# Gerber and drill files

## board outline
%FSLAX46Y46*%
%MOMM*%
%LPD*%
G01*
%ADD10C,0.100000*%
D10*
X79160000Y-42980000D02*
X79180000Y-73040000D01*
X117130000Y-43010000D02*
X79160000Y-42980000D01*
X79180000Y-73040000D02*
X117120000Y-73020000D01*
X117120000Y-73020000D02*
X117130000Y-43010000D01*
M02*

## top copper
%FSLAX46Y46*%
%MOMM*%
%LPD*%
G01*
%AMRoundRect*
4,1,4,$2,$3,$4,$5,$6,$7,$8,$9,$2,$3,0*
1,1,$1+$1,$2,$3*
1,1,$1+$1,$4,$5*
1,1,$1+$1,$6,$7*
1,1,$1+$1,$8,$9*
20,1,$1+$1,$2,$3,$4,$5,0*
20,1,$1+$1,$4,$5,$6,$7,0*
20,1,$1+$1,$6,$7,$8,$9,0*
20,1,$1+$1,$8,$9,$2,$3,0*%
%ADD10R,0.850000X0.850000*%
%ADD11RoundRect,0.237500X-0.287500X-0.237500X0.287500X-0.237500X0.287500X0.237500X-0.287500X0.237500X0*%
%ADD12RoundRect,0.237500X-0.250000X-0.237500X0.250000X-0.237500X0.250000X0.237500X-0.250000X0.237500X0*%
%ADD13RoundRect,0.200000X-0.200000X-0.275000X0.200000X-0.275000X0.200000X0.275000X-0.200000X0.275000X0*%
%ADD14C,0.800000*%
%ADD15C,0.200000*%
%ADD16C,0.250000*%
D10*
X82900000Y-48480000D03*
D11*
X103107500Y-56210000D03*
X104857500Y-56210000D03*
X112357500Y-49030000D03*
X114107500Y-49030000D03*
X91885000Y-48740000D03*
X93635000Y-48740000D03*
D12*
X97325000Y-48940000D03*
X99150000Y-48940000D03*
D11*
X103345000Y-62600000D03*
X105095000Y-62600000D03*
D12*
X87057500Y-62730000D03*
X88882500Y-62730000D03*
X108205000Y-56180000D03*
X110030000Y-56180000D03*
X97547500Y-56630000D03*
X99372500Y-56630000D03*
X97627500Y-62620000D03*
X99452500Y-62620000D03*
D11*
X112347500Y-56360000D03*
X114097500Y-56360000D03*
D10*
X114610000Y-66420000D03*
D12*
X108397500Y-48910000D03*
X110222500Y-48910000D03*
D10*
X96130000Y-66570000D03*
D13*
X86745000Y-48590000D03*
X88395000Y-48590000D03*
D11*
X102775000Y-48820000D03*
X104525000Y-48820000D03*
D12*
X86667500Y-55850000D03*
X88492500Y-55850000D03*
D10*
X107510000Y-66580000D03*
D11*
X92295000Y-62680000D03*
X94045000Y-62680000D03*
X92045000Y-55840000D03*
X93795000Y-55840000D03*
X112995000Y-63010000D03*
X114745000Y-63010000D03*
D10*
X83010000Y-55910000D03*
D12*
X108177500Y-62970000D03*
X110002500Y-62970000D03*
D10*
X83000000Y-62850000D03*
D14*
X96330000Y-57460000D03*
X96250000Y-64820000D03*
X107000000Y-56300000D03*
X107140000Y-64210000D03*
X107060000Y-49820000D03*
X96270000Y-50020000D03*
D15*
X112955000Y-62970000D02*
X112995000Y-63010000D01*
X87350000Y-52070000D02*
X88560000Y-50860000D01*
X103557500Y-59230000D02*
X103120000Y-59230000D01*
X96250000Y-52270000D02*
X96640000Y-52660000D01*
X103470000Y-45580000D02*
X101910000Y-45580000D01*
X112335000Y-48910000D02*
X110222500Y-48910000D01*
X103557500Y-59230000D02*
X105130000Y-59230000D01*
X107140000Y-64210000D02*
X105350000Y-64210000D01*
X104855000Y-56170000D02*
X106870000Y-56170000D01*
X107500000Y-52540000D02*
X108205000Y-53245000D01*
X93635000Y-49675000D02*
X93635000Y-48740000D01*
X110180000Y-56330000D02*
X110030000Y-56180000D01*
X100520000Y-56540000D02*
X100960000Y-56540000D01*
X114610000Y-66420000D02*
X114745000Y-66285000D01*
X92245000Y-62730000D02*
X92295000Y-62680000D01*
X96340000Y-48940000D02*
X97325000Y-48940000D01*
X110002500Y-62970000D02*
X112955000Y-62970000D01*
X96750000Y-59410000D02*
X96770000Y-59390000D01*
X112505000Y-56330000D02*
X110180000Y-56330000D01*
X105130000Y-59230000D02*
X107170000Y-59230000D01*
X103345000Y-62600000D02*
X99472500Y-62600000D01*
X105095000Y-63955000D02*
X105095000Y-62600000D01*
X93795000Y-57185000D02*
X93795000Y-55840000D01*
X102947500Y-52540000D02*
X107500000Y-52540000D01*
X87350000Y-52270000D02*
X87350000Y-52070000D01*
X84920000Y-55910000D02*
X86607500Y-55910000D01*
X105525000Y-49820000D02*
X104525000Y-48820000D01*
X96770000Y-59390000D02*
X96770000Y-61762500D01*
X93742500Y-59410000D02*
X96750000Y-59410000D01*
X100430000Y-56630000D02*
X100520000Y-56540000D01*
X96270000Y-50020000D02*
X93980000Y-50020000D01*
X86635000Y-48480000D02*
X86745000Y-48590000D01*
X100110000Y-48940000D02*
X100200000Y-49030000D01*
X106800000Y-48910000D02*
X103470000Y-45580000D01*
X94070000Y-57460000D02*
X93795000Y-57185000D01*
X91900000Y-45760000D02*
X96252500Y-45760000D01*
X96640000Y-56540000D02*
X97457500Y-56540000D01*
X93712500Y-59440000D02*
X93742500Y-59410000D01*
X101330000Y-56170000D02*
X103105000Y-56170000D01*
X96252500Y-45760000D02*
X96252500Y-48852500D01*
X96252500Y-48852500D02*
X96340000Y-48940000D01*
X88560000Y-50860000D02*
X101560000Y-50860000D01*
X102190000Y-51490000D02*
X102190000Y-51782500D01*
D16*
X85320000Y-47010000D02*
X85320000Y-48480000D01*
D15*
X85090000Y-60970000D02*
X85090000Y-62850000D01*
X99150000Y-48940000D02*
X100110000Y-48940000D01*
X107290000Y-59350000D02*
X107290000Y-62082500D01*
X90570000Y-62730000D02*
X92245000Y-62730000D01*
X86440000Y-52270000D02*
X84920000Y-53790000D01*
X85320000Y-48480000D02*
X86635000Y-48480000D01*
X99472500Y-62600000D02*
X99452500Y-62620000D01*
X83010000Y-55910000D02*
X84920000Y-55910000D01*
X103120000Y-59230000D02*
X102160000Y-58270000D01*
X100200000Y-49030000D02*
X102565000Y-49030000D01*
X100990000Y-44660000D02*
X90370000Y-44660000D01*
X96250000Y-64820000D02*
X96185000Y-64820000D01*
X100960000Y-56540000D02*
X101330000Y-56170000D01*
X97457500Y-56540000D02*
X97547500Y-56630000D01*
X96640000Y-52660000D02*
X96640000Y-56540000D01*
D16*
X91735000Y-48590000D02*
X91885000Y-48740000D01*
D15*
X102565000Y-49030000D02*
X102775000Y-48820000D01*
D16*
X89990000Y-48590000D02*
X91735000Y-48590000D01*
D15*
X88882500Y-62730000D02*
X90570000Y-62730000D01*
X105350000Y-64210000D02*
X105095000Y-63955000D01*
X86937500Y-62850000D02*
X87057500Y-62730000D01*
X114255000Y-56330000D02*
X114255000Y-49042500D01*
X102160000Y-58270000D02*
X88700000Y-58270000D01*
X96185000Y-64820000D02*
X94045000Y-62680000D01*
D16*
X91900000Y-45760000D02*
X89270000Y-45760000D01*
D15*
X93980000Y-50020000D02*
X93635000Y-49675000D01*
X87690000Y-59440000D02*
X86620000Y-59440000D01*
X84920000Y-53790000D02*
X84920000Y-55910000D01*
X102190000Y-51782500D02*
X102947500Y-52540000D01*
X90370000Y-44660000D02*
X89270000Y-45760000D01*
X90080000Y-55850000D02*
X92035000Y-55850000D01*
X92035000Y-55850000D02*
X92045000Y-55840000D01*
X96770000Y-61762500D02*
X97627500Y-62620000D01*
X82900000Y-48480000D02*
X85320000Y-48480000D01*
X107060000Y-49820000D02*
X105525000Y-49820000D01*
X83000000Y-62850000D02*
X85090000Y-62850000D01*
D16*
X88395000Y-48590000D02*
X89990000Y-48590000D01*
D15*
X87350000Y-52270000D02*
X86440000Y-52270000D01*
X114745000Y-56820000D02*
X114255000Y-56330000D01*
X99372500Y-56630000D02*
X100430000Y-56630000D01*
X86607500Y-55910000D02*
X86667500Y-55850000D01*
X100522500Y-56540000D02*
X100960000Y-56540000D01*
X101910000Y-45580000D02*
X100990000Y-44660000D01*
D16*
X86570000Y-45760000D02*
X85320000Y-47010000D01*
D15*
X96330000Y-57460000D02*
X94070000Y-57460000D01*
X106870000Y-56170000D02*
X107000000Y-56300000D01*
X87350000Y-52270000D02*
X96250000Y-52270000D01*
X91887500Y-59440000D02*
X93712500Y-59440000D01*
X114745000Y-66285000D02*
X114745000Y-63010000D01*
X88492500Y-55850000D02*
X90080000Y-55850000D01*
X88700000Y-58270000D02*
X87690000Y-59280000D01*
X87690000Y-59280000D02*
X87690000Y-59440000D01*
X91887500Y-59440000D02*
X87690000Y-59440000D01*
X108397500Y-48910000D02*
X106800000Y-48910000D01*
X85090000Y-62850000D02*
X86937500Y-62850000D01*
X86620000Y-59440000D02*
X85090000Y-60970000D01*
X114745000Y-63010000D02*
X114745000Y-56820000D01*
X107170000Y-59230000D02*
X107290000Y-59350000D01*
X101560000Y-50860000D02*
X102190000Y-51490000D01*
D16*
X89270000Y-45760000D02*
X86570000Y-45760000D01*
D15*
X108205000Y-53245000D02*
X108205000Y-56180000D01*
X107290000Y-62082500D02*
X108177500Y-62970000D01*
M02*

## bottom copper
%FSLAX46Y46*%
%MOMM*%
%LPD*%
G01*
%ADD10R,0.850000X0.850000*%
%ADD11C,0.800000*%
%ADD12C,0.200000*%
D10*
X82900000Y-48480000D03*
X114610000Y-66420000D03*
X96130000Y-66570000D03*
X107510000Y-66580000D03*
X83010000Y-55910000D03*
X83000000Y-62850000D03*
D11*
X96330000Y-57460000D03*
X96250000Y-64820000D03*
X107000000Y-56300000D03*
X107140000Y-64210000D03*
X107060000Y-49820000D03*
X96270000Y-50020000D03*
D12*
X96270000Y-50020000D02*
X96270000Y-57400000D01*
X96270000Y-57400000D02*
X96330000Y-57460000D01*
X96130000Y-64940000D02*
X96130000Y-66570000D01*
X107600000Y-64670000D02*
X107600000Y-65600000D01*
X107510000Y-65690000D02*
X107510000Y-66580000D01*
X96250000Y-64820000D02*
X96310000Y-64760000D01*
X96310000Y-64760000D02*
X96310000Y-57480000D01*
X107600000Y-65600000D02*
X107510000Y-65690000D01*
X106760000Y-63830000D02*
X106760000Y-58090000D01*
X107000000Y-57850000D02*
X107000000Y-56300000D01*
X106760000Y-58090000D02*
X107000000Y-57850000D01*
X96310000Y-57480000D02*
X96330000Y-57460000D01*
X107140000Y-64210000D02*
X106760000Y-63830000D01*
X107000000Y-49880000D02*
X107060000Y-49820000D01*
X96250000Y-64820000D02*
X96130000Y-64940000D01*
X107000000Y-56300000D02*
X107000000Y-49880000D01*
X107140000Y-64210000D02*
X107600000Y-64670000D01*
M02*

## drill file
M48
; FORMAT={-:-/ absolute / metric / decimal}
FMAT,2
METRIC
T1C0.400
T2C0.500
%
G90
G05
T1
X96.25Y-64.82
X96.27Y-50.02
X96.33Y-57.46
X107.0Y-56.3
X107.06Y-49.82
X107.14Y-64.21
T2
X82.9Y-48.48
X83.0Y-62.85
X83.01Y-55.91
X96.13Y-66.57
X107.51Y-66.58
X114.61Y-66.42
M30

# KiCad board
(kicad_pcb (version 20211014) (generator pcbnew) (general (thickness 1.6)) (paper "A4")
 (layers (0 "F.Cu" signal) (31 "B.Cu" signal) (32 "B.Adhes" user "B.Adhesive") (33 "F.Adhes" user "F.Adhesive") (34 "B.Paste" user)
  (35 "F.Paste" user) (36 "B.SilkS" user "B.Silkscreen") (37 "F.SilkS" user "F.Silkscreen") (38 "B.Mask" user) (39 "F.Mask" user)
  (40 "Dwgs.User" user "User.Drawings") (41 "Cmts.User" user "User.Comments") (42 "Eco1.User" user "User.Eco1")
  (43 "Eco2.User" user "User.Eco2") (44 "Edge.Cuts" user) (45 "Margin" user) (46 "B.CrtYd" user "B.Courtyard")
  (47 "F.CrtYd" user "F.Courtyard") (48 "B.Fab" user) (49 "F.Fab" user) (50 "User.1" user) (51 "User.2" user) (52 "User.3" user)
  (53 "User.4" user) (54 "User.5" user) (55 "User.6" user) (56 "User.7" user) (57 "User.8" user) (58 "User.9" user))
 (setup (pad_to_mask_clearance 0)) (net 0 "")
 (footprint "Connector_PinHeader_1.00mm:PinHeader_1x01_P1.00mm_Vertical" (layer "F.Cu") (at 82.9 48.48)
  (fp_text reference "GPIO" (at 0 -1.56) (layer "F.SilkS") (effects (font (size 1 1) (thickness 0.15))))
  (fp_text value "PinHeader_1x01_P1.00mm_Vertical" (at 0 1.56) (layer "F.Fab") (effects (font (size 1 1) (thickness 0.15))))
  (pad "1" thru_hole rect (at 0 0) (size 0.85 0.85) (drill 0.5) (layers *.Cu *.Mask)))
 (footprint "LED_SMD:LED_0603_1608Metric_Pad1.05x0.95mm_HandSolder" (layer "F.Cu") (at 103.9825 56.21)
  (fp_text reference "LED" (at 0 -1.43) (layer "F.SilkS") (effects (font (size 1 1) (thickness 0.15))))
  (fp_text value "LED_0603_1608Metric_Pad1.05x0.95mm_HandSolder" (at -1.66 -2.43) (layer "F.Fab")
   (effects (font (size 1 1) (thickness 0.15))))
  (pad "1" smd roundrect (at -0.875 0) (size 1.05 0.95) (layers "F.Cu" "F.Paste" "F.Mask") (roundrect_rratio 0.25))
  (pad "2" smd roundrect (at 0.875 0) (size 1.05 0.95) (layers "F.Cu" "F.Paste" "F.Mask") (roundrect_rratio 0.25)))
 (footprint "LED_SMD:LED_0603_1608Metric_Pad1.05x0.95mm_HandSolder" (layer "F.Cu") (at 113.2325 49.03)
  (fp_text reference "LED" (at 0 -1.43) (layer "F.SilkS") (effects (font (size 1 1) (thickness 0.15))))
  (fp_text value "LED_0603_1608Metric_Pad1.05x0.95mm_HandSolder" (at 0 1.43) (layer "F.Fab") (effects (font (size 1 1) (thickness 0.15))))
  (pad "1" smd roundrect (at -0.875 0) (size 1.05 0.95) (layers "F.Cu" "F.Paste" "F.Mask") (roundrect_rratio 0.25))
  (pad "2" smd roundrect (at 0.875 0) (size 1.05 0.95) (layers "F.Cu" "F.Paste" "F.Mask") (roundrect_rratio 0.25)))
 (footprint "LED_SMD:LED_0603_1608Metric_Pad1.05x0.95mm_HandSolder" (layer "F.Cu") (at 92.76 48.74)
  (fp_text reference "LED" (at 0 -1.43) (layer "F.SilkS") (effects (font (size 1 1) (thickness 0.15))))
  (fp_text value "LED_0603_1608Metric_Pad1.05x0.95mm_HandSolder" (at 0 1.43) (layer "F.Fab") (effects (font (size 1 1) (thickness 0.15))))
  (pad "1" smd roundrect (at -0.875 0) (size 1.05 0.95) (layers "F.Cu" "F.Paste" "F.Mask") (roundrect_rratio 0.25))
  (pad "2" smd roundrect (at 0.875 0) (size 1.05 0.95) (layers "F.Cu" "F.Paste" "F.Mask") (roundrect_rratio 0.25)))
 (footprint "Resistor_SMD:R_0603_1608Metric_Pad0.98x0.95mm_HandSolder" (layer "F.Cu") (at 98.2375 48.94)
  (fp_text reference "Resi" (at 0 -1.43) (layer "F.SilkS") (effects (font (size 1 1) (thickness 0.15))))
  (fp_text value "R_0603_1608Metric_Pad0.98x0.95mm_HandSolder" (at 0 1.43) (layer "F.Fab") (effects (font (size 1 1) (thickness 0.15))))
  (pad "1" smd roundrect (at -0.9125 0) (size 0.975 0.95) (layers "F.Cu" "F.Paste" "F.Mask") (roundrect_rratio 0.25))
  (pad "2" smd roundrect (at 0.9125 0) (size 0.975 0.95) (layers "F.Cu" "F.Paste" "F.Mask") (roundrect_rratio 0.25)))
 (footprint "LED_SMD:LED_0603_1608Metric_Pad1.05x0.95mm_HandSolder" (layer "F.Cu") (at 104.22 62.6)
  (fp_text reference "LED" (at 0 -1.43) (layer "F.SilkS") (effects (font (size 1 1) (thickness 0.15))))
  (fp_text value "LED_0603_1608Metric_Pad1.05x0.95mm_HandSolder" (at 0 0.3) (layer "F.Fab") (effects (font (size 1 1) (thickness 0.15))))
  (pad "1" smd roundrect (at -0.875 0) (size 1.05 0.95) (layers "F.Cu" "F.Paste" "F.Mask") (roundrect_rratio 0.25))
  (pad "2" smd roundrect (at 0.875 0) (size 1.05 0.95) (layers "F.Cu" "F.Paste" "F.Mask") (roundrect_rratio 0.25)))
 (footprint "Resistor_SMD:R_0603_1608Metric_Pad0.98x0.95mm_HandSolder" (layer "F.Cu") (at 87.97 62.73)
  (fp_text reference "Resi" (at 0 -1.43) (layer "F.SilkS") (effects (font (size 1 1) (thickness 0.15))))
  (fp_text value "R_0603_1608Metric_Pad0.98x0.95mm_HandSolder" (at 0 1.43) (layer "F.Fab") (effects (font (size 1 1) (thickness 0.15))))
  (pad "1" smd roundrect (at -0.9125 0) (size 0.975 0.95) (layers "F.Cu" "F.Paste" "F.Mask") (roundrect_rratio 0.25))
  (pad "2" smd roundrect (at 0.9125 0) (size 0.975 0.95) (layers "F.Cu" "F.Paste" "F.Mask") (roundrect_rratio 0.25)))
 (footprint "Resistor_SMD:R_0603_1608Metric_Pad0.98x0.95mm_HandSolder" (layer "F.Cu") (at 109.1175 56.18)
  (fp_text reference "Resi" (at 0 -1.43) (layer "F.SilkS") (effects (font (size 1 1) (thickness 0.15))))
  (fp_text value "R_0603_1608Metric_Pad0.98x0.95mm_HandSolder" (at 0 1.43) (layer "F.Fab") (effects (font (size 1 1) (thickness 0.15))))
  (pad "1" smd roundrect (at -0.9125 0) (size 0.975 0.95) (layers "F.Cu" "F.Paste" "F.Mask") (roundrect_rratio 0.25))
  (pad "2" smd roundrect (at 0.9125 0) (size 0.975 0.95) (layers "F.Cu" "F.Paste" "F.Mask") (roundrect_rratio 0.25)))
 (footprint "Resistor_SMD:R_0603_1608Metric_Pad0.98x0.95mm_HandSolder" (layer "F.Cu") (at 98.46 56.63)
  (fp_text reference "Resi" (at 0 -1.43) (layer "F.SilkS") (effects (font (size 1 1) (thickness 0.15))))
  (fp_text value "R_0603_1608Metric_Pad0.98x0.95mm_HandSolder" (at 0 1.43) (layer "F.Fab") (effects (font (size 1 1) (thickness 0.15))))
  (pad "1" smd roundrect (at -0.9125 0) (size 0.975 0.95) (layers "F.Cu" "F.Paste" "F.Mask") (roundrect_rratio 0.25))
  (pad "2" smd roundrect (at 0.9125 0) (size 0.975 0.95) (layers "F.Cu" "F.Paste" "F.Mask") (roundrect_rratio 0.25)))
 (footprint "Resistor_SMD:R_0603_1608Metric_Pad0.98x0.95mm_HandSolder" (layer "F.Cu") (at 98.54 62.62)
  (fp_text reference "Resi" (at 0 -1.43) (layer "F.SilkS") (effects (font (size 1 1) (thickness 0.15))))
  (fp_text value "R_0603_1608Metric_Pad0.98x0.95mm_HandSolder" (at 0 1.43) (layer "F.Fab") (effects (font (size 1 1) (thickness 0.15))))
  (pad "1" smd roundrect (at -0.9125 0) (size 0.975 0.95) (layers "F.Cu" "F.Paste" "F.Mask") (roundrect_rratio 0.25))
  (pad "2" smd roundrect (at 0.9125 0) (size 0.975 0.95) (layers "F.Cu" "F.Paste" "F.Mask") (roundrect_rratio 0.25)))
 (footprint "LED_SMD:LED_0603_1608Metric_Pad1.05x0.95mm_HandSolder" (layer "F.Cu") (at 113.2225 56.36)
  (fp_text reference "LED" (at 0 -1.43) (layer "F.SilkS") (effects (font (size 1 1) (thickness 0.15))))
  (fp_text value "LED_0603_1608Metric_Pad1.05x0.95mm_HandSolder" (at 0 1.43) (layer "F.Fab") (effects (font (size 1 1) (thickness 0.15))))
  (pad "1" smd roundrect (at -0.875 0) (size 1.05 0.95) (layers "F.Cu" "F.Paste" "F.Mask") (roundrect_rratio 0.25))
  (pad "2" smd roundrect (at 0.875 0) (size 1.05 0.95) (layers "F.Cu" "F.Paste" "F.Mask") (roundrect_rratio 0.25)))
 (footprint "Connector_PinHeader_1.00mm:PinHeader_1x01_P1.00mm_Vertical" (layer "F.Cu") (at 114.61 66.42)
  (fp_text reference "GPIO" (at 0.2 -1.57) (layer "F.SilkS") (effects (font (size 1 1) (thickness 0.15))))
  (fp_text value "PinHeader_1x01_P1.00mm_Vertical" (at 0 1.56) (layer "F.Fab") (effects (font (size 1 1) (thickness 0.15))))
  (pad "1" thru_hole rect (at 0 0) (size 0.85 0.85) (drill 0.5) (layers *.Cu *.Mask)))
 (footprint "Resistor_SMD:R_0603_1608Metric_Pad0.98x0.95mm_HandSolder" (layer "F.Cu") (at 109.31 48.91)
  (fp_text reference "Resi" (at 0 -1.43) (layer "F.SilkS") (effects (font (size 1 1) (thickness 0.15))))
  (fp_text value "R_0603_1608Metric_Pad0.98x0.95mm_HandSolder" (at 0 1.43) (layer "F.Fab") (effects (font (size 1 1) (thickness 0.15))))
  (pad "1" smd roundrect (at -0.9125 0) (size 0.975 0.95) (layers "F.Cu" "F.Paste" "F.Mask") (roundrect_rratio 0.25))
  (pad "2" smd roundrect (at 0.9125 0) (size 0.975 0.95) (layers "F.Cu" "F.Paste" "F.Mask") (roundrect_rratio 0.25)))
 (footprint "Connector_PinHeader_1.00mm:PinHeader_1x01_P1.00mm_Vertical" (layer "F.Cu") (at 96.13 66.57)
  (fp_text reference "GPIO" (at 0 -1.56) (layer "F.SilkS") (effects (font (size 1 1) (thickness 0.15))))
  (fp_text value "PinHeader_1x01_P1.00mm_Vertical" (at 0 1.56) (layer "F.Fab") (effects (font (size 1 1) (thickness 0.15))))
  (pad "1" thru_hole rect (at 0 0) (size 0.85 0.85) (drill 0.5) (layers *.Cu *.Mask)))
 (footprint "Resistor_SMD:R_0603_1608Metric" (layer "F.Cu") (at 87.57 48.59)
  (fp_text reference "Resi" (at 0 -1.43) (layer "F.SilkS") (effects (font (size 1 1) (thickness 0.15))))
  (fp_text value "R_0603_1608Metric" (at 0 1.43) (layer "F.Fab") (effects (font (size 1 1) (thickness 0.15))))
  (pad "1" smd roundrect (at -0.825 0) (size 0.8 0.95) (layers "F.Cu" "F.Paste" "F.Mask") (roundrect_rratio 0.25))
  (pad "2" smd roundrect (at 0.825 0) (size 0.8 0.95) (layers "F.Cu" "F.Paste" "F.Mask") (roundrect_rratio 0.25)))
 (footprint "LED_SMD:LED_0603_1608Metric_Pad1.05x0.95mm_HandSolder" (layer "F.Cu") (at 103.65 48.82)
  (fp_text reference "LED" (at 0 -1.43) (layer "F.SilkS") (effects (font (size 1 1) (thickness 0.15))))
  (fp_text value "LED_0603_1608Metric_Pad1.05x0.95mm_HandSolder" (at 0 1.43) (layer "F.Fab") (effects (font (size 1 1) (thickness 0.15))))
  (pad "1" smd roundrect (at -0.875 0) (size 1.05 0.95) (layers "F.Cu" "F.Paste" "F.Mask") (roundrect_rratio 0.25))
  (pad "2" smd roundrect (at 0.875 0) (size 1.05 0.95) (layers "F.Cu" "F.Paste" "F.Mask") (roundrect_rratio 0.25)))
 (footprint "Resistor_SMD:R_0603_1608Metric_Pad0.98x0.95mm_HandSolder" (layer "F.Cu") (at 87.58 55.85)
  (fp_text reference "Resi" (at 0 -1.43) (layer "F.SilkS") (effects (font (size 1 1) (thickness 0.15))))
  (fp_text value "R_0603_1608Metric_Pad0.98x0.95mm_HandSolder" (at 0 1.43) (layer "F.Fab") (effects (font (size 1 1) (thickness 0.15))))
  (pad "1" smd roundrect (at -0.9125 0) (size 0.975 0.95) (layers "F.Cu" "F.Paste" "F.Mask") (roundrect_rratio 0.25))
  (pad "2" smd roundrect (at 0.9125 0) (size 0.975 0.95) (layers "F.Cu" "F.Paste" "F.Mask") (roundrect_rratio 0.25)))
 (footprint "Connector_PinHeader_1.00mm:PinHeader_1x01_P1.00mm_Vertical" (layer "F.Cu") (at 107.51 66.58)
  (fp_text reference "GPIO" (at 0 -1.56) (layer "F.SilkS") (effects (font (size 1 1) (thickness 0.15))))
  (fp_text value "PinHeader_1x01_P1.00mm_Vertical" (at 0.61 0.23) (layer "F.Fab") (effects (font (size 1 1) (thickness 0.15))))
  (pad "1" thru_hole rect (at 0 0) (size 0.85 0.85) (drill 0.5) (layers *.Cu *.Mask)))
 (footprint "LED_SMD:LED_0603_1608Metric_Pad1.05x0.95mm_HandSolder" (layer "F.Cu") (at 93.17 62.68)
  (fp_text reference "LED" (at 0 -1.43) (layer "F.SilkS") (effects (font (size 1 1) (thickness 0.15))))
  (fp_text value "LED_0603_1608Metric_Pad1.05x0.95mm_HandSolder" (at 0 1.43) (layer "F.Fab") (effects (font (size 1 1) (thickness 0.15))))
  (pad "1" smd roundrect (at -0.875 0) (size 1.05 0.95) (layers "F.Cu" "F.Paste" "F.Mask") (roundrect_rratio 0.25))
  (pad "2" smd roundrect (at 0.875 0) (size 1.05 0.95) (layers "F.Cu" "F.Paste" "F.Mask") (roundrect_rratio 0.25)))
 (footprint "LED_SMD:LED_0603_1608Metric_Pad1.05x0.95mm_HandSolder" (layer "F.Cu") (at 92.92 55.84)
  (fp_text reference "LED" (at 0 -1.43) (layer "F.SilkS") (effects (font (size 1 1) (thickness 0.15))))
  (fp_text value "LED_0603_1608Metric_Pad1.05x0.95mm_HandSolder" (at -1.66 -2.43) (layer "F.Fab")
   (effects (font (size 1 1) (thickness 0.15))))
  (pad "1" smd roundrect (at -0.875 0) (size 1.05 0.95) (layers "F.Cu" "F.Paste" "F.Mask") (roundrect_rratio 0.25))
  (pad "2" smd roundrect (at 0.875 0) (size 1.05 0.95) (layers "F.Cu" "F.Paste" "F.Mask") (roundrect_rratio 0.25)))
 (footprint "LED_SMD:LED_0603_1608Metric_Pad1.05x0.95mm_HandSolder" (layer "F.Cu") (at 113.87 63.01)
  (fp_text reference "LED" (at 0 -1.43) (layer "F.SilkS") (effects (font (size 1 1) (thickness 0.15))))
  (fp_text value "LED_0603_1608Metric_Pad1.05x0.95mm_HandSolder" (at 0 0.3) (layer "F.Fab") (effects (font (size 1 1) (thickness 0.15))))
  (pad "1" smd roundrect (at -0.875 0) (size 1.05 0.95) (layers "F.Cu" "F.Paste" "F.Mask") (roundrect_rratio 0.25))
  (pad "2" smd roundrect (at 0.875 0) (size 1.05 0.95) (layers "F.Cu" "F.Paste" "F.Mask") (roundrect_rratio 0.25)))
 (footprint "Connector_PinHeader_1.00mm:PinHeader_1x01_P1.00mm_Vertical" (layer "F.Cu") (at 83.01 55.91)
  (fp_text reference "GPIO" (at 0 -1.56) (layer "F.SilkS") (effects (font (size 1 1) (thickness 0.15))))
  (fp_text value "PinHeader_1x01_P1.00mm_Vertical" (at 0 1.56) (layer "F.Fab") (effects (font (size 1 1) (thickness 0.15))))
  (pad "1" thru_hole rect (at 0 0) (size 0.85 0.85) (drill 0.5) (layers *.Cu *.Mask)))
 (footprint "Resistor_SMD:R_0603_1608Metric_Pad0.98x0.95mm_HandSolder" (layer "F.Cu") (at 109.09 62.97)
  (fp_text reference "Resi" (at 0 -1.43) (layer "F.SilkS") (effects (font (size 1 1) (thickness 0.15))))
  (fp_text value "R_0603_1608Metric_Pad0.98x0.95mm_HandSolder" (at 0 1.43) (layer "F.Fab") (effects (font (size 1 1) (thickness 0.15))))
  (pad "1" smd roundrect (at -0.9125 0) (size 0.975 0.95) (layers "F.Cu" "F.Paste" "F.Mask") (roundrect_rratio 0.25))
  (pad "2" smd roundrect (at 0.9125 0) (size 0.975 0.95) (layers "F.Cu" "F.Paste" "F.Mask") (roundrect_rratio 0.25)))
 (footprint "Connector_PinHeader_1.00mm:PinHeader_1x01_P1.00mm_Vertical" (layer "F.Cu") (at 83 62.85)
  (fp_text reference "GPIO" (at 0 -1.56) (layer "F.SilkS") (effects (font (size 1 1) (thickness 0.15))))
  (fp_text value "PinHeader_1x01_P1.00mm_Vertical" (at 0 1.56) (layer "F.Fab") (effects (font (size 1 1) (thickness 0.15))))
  (pad "1" thru_hole rect (at 0 0) (size 0.85 0.85) (drill 0.5) (layers *.Cu *.Mask)))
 (gr_line (start 79.16 42.98) (end 79.18 73.04) (layer "Edge.Cuts") (width 0.1))
 (gr_line (start 117.13 43.01) (end 79.16 42.98) (layer "Edge.Cuts") (width 0.1))
 (gr_line (start 79.18 73.04) (end 117.12 73.02) (layer "Edge.Cuts") (width 0.1))
 (gr_line (start 117.12 73.02) (end 117.13 43.01) (layer "Edge.Cuts") (width 0.1))
 (segment (start 112.955 62.97) (end 112.995 63.01) (width 0.2) (layer "F.Cu") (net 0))
 (segment (start 87.35 52.07) (end 88.56 50.86) (width 0.2) (layer "F.Cu") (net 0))
 (segment (start 103.5575 59.23) (end 103.12 59.23) (width 0.2) (layer "F.Cu") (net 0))
 (segment (start 96.25 52.27) (end 96.64 52.66) (width 0.2) (layer "F.Cu") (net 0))
 (segment (start 103.47 45.58) (end 101.91 45.58) (width 0.2) (layer "F.Cu") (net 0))
 (segment (start 112.335 48.91) (end 110.2225 48.91) (width 0.2) (layer "F.Cu") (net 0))
 (segment (start 103.5575 59.23) (end 105.13 59.23) (width 0.2) (layer "F.Cu") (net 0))
 (segment (start 107.14 64.21) (end 105.35 64.21) (width 0.2) (layer "F.Cu") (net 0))
 (segment (start 104.855 56.17) (end 106.87 56.17) (width 0.2) (layer "F.Cu") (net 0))
 (segment (start 107.5 52.54) (end 108.205 53.245) (width 0.2) (layer "F.Cu") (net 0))
 (segment (start 93.635 49.675) (end 93.635 48.74) (width 0.2) (layer "F.Cu") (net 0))
 (segment (start 110.18 56.33) (end 110.03 56.18) (width 0.2) (layer "F.Cu") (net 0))
 (segment (start 100.52 56.54) (end 100.96 56.54) (width 0.2) (layer "F.Cu") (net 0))
 (segment (start 114.61 66.42) (end 114.745 66.285) (width 0.2) (layer "F.Cu") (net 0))
 (segment (start 92.245 62.73) (end 92.295 62.68) (width 0.2) (layer "F.Cu") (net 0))
 (segment (start 96.34 48.94) (end 97.325 48.94) (width 0.2) (layer "F.Cu") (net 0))
 (segment (start 110.0025 62.97) (end 112.955 62.97) (width 0.2) (layer "F.Cu") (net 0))
 (segment (start 96.75 59.41) (end 96.77 59.39) (width 0.2) (layer "F.Cu") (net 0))
 (segment (start 112.505 56.33) (end 110.18 56.33) (width 0.2) (layer "F.Cu") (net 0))
 (segment (start 105.13 59.23) (end 107.17 59.23) (width 0.2) (layer "F.Cu") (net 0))
 (segment (start 103.345 62.6) (end 99.4725 62.6) (width 0.2) (layer "F.Cu") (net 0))
 (segment (start 105.095 63.955) (end 105.095 62.6) (width 0.2) (layer "F.Cu") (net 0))
 (segment (start 93.795 57.185) (end 93.795 55.84) (width 0.2) (layer "F.Cu") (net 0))
 (segment (start 102.9475 52.54) (end 107.5 52.54) (width 0.2) (layer "F.Cu") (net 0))
 (segment (start 87.35 52.27) (end 87.35 52.07) (width 0.2) (layer "F.Cu") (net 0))
 (segment (start 84.92 55.91) (end 86.6075 55.91) (width 0.2) (layer "F.Cu") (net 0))
 (segment (start 105.525 49.82) (end 104.525 48.82) (width 0.2) (layer "F.Cu") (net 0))
 (segment (start 96.77 59.39) (end 96.77 61.7625) (width 0.2) (layer "F.Cu") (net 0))
 (segment (start 93.7425 59.41) (end 96.75 59.41) (width 0.2) (layer "F.Cu") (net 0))
 (segment (start 100.43 56.63) (end 100.52 56.54) (width 0.2) (layer "F.Cu") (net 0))
 (segment (start 96.27 50.02) (end 93.98 50.02) (width 0.2) (layer "F.Cu") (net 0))
 (segment (start 86.635 48.48) (end 86.745 48.59) (width 0.2) (layer "F.Cu") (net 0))
 (segment (start 100.11 48.94) (end 100.2 49.03) (width 0.2) (layer "F.Cu") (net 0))
 (segment (start 106.8 48.91) (end 103.47 45.58) (width 0.2) (layer "F.Cu") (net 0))
 (segment (start 94.07 57.46) (end 93.795 57.185) (width 0.2) (layer "F.Cu") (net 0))
 (segment (start 91.9 45.76) (end 96.2525 45.76) (width 0.2) (layer "F.Cu") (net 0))
 (segment (start 96.64 56.54) (end 97.4575 56.54) (width 0.2) (layer "F.Cu") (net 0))
 (segment (start 93.7125 59.44) (end 93.7425 59.41) (width 0.2) (layer "F.Cu") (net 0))
 (segment (start 101.33 56.17) (end 103.105 56.17) (width 0.2) (layer "F.Cu") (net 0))
 (segment (start 96.2525 45.76) (end 96.2525 48.8525) (width 0.2) (layer "F.Cu") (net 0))
 (segment (start 96.2525 48.8525) (end 96.34 48.94) (width 0.2) (layer "F.Cu") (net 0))
 (segment (start 88.56 50.86) (end 101.56 50.86) (width 0.2) (layer "F.Cu") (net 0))
 (segment (start 102.19 51.49) (end 102.19 51.7825) (width 0.2) (layer "F.Cu") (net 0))
 (segment (start 85.32 47.01) (end 85.32 48.48) (width 0.25) (layer "F.Cu") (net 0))
 (segment (start 85.09 60.97) (end 85.09 62.85) (width 0.2) (layer "F.Cu") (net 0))
 (segment (start 99.15 48.94) (end 100.11 48.94) (width 0.2) (layer "F.Cu") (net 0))
 (segment (start 107.29 59.35) (end 107.29 62.0825) (width 0.2) (layer "F.Cu") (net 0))
 (segment (start 90.57 62.73) (end 92.245 62.73) (width 0.2) (layer "F.Cu") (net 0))
 (segment (start 86.44 52.27) (end 84.92 53.79) (width 0.2) (layer "F.Cu") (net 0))
 (segment (start 85.32 48.48) (end 86.635 48.48) (width 0.2) (layer "F.Cu") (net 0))
 (segment (start 99.4725 62.6) (end 99.4525 62.62) (width 0.2) (layer "F.Cu") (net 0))
 (segment (start 83.01 55.91) (end 84.92 55.91) (width 0.2) (layer "F.Cu") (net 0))
 (segment (start 103.12 59.23) (end 102.16 58.27) (width 0.2) (layer "F.Cu") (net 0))
 (segment (start 100.2 49.03) (end 102.565 49.03) (width 0.2) (layer "F.Cu") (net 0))
 (segment (start 100.99 44.66) (end 90.37 44.66) (width 0.2) (layer "F.Cu") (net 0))
 (segment (start 96.25 64.82) (end 96.185 64.82) (width 0.2) (layer "F.Cu") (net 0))
 (segment (start 100.96 56.54) (end 101.33 56.17) (width 0.2) (layer "F.Cu") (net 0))
 (segment (start 97.4575 56.54) (end 97.5475 56.63) (width 0.2) (layer "F.Cu") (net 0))
 (segment (start 96.64 52.66) (end 96.64 56.54) (width 0.2) (layer "F.Cu") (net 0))
 (segment (start 91.735 48.59) (end 91.885 48.74) (width 0.25) (layer "F.Cu") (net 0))
 (segment (start 102.565 49.03) (end 102.775 48.82) (width 0.2) (layer "F.Cu") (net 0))
 (segment (start 89.99 48.59) (end 91.735 48.59) (width 0.25) (layer "F.Cu") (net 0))
 (segment (start 88.8825 62.73) (end 90.57 62.73) (width 0.2) (layer "F.Cu") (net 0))
 (segment (start 105.35 64.21) (end 105.095 63.955) (width 0.2) (layer "F.Cu") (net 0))
 (segment (start 86.9375 62.85) (end 87.0575 62.73) (width 0.2) (layer "F.Cu") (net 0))
 (segment (start 114.255 56.33) (end 114.255 49.0425) (width 0.2) (layer "F.Cu") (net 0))
 (segment (start 102.16 58.27) (end 88.7 58.27) (width 0.2) (layer "F.Cu") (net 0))
 (segment (start 96.185 64.82) (end 94.045 62.68) (width 0.2) (layer "F.Cu") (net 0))
 (segment (start 91.9 45.76) (end 89.27 45.76) (width 0.25) (layer "F.Cu") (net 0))
 (segment (start 93.98 50.02) (end 93.635 49.675) (width 0.2) (layer "F.Cu") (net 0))
 (segment (start 87.69 59.44) (end 86.62 59.44) (width 0.2) (layer "F.Cu") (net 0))
 (segment (start 84.92 53.79) (end 84.92 55.91) (width 0.2) (layer "F.Cu") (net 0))
 (segment (start 102.19 51.7825) (end 102.9475 52.54) (width 0.2) (layer "F.Cu") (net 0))
 (segment (start 90.37 44.66) (end 89.27 45.76) (width 0.2) (layer "F.Cu") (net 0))
 (segment (start 90.08 55.85) (end 92.035 55.85) (width 0.2) (layer "F.Cu") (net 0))
 (segment (start 92.035 55.85) (end 92.045 55.84) (width 0.2) (layer "F.Cu") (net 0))
 (segment (start 96.77 61.7625) (end 97.6275 62.62) (width 0.2) (layer "F.Cu") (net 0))
 (segment (start 82.9 48.48) (end 85.32 48.48) (width 0.2) (layer "F.Cu") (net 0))
 (segment (start 107.06 49.82) (end 105.525 49.82) (width 0.2) (layer "F.Cu") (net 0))
 (segment (start 83 62.85) (end 85.09 62.85) (width 0.2) (layer "F.Cu") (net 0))
 (segment (start 88.395 48.59) (end 89.99 48.59) (width 0.25) (layer "F.Cu") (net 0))
 (segment (start 87.35 52.27) (end 86.44 52.27) (width 0.2) (layer "F.Cu") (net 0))
 (segment (start 114.745 56.82) (end 114.255 56.33) (width 0.2) (layer "F.Cu") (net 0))
 (segment (start 99.3725 56.63) (end 100.43 56.63) (width 0.2) (layer "F.Cu") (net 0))
 (segment (start 86.6075 55.91) (end 86.6675 55.85) (width 0.2) (layer "F.Cu") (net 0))
 (segment (start 100.5225 56.54) (end 100.96 56.54) (width 0.2) (layer "F.Cu") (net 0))
 (segment (start 101.91 45.58) (end 100.99 44.66) (width 0.2) (layer "F.Cu") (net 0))
 (segment (start 86.57 45.76) (end 85.32 47.01) (width 0.25) (layer "F.Cu") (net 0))
 (segment (start 96.33 57.46) (end 94.07 57.46) (width 0.2) (layer "F.Cu") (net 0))
 (segment (start 106.87 56.17) (end 107 56.3) (width 0.2) (layer "F.Cu") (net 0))
 (segment (start 87.35 52.27) (end 96.25 52.27) (width 0.2) (layer "F.Cu") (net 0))
 (segment (start 91.8875 59.44) (end 93.7125 59.44) (width 0.2) (layer "F.Cu") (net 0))
 (segment (start 114.745 66.285) (end 114.745 63.01) (width 0.2) (layer "F.Cu") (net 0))
 (segment (start 88.4925 55.85) (end 90.08 55.85) (width 0.2) (layer "F.Cu") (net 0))
 (segment (start 88.7 58.27) (end 87.69 59.28) (width 0.2) (layer "F.Cu") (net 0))
 (segment (start 87.69 59.28) (end 87.69 59.44) (width 0.2) (layer "F.Cu") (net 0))
 (segment (start 91.8875 59.44) (end 87.69 59.44) (width 0.2) (layer "F.Cu") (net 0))
 (segment (start 108.3975 48.91) (end 106.8 48.91) (width 0.2) (layer "F.Cu") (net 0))
 (segment (start 85.09 62.85) (end 86.9375 62.85) (width 0.2) (layer "F.Cu") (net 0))
 (segment (start 86.62 59.44) (end 85.09 60.97) (width 0.2) (layer "F.Cu") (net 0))
 (segment (start 114.745 63.01) (end 114.745 56.82) (width 0.2) (layer "F.Cu") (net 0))
 (segment (start 107.17 59.23) (end 107.29 59.35) (width 0.2) (layer "F.Cu") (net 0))
 (segment (start 101.56 50.86) (end 102.19 51.49) (width 0.2) (layer "F.Cu") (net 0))
 (segment (start 89.27 45.76) (end 86.57 45.76) (width 0.25) (layer "F.Cu") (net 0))
 (segment (start 108.205 53.245) (end 108.205 56.18) (width 0.2) (layer "F.Cu") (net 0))
 (segment (start 107.29 62.0825) (end 108.1775 62.97) (width 0.2) (layer "F.Cu") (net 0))
 (via (at 96.33 57.46) (size 0.8) (drill 0.4) (layers "F.Cu" "B.Cu") (free) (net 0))
 (via (at 96.25 64.82) (size 0.8) (drill 0.4) (layers "F.Cu" "B.Cu") (free) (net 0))
 (via (at 107 56.3) (size 0.8) (drill 0.4) (layers "F.Cu" "B.Cu") (free) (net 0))
 (via (at 107.14 64.21) (size 0.8) (drill 0.4) (layers "F.Cu" "B.Cu") (free) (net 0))
 (via (at 107.06 49.82) (size 0.8) (drill 0.4) (layers "F.Cu" "B.Cu") (free) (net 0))
 (via (at 96.27 50.02) (size 0.8) (drill 0.4) (layers "F.Cu" "B.Cu") (free) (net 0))
 (segment (start 96.27 50.02) (end 96.27 57.4) (width 0.2) (layer "B.Cu") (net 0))
 (segment (start 96.27 57.4) (end 96.33 57.46) (width 0.2) (layer "B.Cu") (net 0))
 (segment (start 96.13 64.94) (end 96.13 66.57) (width 0.2) (layer "B.Cu") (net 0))
 (segment (start 107.6 64.67) (end 107.6 65.6) (width 0.2) (layer "B.Cu") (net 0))
 (segment (start 107.51 65.69) (end 107.51 66.58) (width 0.2) (layer "B.Cu") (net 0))
 (segment (start 96.25 64.82) (end 96.31 64.76) (width 0.2) (layer "B.Cu") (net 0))
 (segment (start 96.31 64.76) (end 96.31 57.48) (width 0.2) (layer "B.Cu") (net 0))
 (segment (start 107.6 65.6) (end 107.51 65.69) (width 0.2) (layer "B.Cu") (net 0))
 (segment (start 106.76 63.83) (end 106.76 58.09) (width 0.2) (layer "B.Cu") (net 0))
 (segment (start 107 57.85) (end 107 56.3) (width 0.2) (layer "B.Cu") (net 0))
 (segment (start 106.76 58.09) (end 107 57.85) (width 0.2) (layer "B.Cu") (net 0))
 (segment (start 96.31 57.48) (end 96.33 57.46) (width 0.2) (layer "B.Cu") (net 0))
 (segment (start 107.14 64.21) (end 106.76 63.83) (width 0.2) (layer "B.Cu") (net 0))
 (segment (start 107 49.88) (end 107.06 49.82) (width 0.2) (layer "B.Cu") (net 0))
 (segment (start 96.25 64.82) (end 96.13 64.94) (width 0.2) (layer "B.Cu") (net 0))
 (segment (start 107 56.3) (end 107 49.88) (width 0.2) (layer "B.Cu") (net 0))
 (segment (start 107.14 64.21) (end 107.6 64.67) (width 0.2) (layer "B.Cu") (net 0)))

